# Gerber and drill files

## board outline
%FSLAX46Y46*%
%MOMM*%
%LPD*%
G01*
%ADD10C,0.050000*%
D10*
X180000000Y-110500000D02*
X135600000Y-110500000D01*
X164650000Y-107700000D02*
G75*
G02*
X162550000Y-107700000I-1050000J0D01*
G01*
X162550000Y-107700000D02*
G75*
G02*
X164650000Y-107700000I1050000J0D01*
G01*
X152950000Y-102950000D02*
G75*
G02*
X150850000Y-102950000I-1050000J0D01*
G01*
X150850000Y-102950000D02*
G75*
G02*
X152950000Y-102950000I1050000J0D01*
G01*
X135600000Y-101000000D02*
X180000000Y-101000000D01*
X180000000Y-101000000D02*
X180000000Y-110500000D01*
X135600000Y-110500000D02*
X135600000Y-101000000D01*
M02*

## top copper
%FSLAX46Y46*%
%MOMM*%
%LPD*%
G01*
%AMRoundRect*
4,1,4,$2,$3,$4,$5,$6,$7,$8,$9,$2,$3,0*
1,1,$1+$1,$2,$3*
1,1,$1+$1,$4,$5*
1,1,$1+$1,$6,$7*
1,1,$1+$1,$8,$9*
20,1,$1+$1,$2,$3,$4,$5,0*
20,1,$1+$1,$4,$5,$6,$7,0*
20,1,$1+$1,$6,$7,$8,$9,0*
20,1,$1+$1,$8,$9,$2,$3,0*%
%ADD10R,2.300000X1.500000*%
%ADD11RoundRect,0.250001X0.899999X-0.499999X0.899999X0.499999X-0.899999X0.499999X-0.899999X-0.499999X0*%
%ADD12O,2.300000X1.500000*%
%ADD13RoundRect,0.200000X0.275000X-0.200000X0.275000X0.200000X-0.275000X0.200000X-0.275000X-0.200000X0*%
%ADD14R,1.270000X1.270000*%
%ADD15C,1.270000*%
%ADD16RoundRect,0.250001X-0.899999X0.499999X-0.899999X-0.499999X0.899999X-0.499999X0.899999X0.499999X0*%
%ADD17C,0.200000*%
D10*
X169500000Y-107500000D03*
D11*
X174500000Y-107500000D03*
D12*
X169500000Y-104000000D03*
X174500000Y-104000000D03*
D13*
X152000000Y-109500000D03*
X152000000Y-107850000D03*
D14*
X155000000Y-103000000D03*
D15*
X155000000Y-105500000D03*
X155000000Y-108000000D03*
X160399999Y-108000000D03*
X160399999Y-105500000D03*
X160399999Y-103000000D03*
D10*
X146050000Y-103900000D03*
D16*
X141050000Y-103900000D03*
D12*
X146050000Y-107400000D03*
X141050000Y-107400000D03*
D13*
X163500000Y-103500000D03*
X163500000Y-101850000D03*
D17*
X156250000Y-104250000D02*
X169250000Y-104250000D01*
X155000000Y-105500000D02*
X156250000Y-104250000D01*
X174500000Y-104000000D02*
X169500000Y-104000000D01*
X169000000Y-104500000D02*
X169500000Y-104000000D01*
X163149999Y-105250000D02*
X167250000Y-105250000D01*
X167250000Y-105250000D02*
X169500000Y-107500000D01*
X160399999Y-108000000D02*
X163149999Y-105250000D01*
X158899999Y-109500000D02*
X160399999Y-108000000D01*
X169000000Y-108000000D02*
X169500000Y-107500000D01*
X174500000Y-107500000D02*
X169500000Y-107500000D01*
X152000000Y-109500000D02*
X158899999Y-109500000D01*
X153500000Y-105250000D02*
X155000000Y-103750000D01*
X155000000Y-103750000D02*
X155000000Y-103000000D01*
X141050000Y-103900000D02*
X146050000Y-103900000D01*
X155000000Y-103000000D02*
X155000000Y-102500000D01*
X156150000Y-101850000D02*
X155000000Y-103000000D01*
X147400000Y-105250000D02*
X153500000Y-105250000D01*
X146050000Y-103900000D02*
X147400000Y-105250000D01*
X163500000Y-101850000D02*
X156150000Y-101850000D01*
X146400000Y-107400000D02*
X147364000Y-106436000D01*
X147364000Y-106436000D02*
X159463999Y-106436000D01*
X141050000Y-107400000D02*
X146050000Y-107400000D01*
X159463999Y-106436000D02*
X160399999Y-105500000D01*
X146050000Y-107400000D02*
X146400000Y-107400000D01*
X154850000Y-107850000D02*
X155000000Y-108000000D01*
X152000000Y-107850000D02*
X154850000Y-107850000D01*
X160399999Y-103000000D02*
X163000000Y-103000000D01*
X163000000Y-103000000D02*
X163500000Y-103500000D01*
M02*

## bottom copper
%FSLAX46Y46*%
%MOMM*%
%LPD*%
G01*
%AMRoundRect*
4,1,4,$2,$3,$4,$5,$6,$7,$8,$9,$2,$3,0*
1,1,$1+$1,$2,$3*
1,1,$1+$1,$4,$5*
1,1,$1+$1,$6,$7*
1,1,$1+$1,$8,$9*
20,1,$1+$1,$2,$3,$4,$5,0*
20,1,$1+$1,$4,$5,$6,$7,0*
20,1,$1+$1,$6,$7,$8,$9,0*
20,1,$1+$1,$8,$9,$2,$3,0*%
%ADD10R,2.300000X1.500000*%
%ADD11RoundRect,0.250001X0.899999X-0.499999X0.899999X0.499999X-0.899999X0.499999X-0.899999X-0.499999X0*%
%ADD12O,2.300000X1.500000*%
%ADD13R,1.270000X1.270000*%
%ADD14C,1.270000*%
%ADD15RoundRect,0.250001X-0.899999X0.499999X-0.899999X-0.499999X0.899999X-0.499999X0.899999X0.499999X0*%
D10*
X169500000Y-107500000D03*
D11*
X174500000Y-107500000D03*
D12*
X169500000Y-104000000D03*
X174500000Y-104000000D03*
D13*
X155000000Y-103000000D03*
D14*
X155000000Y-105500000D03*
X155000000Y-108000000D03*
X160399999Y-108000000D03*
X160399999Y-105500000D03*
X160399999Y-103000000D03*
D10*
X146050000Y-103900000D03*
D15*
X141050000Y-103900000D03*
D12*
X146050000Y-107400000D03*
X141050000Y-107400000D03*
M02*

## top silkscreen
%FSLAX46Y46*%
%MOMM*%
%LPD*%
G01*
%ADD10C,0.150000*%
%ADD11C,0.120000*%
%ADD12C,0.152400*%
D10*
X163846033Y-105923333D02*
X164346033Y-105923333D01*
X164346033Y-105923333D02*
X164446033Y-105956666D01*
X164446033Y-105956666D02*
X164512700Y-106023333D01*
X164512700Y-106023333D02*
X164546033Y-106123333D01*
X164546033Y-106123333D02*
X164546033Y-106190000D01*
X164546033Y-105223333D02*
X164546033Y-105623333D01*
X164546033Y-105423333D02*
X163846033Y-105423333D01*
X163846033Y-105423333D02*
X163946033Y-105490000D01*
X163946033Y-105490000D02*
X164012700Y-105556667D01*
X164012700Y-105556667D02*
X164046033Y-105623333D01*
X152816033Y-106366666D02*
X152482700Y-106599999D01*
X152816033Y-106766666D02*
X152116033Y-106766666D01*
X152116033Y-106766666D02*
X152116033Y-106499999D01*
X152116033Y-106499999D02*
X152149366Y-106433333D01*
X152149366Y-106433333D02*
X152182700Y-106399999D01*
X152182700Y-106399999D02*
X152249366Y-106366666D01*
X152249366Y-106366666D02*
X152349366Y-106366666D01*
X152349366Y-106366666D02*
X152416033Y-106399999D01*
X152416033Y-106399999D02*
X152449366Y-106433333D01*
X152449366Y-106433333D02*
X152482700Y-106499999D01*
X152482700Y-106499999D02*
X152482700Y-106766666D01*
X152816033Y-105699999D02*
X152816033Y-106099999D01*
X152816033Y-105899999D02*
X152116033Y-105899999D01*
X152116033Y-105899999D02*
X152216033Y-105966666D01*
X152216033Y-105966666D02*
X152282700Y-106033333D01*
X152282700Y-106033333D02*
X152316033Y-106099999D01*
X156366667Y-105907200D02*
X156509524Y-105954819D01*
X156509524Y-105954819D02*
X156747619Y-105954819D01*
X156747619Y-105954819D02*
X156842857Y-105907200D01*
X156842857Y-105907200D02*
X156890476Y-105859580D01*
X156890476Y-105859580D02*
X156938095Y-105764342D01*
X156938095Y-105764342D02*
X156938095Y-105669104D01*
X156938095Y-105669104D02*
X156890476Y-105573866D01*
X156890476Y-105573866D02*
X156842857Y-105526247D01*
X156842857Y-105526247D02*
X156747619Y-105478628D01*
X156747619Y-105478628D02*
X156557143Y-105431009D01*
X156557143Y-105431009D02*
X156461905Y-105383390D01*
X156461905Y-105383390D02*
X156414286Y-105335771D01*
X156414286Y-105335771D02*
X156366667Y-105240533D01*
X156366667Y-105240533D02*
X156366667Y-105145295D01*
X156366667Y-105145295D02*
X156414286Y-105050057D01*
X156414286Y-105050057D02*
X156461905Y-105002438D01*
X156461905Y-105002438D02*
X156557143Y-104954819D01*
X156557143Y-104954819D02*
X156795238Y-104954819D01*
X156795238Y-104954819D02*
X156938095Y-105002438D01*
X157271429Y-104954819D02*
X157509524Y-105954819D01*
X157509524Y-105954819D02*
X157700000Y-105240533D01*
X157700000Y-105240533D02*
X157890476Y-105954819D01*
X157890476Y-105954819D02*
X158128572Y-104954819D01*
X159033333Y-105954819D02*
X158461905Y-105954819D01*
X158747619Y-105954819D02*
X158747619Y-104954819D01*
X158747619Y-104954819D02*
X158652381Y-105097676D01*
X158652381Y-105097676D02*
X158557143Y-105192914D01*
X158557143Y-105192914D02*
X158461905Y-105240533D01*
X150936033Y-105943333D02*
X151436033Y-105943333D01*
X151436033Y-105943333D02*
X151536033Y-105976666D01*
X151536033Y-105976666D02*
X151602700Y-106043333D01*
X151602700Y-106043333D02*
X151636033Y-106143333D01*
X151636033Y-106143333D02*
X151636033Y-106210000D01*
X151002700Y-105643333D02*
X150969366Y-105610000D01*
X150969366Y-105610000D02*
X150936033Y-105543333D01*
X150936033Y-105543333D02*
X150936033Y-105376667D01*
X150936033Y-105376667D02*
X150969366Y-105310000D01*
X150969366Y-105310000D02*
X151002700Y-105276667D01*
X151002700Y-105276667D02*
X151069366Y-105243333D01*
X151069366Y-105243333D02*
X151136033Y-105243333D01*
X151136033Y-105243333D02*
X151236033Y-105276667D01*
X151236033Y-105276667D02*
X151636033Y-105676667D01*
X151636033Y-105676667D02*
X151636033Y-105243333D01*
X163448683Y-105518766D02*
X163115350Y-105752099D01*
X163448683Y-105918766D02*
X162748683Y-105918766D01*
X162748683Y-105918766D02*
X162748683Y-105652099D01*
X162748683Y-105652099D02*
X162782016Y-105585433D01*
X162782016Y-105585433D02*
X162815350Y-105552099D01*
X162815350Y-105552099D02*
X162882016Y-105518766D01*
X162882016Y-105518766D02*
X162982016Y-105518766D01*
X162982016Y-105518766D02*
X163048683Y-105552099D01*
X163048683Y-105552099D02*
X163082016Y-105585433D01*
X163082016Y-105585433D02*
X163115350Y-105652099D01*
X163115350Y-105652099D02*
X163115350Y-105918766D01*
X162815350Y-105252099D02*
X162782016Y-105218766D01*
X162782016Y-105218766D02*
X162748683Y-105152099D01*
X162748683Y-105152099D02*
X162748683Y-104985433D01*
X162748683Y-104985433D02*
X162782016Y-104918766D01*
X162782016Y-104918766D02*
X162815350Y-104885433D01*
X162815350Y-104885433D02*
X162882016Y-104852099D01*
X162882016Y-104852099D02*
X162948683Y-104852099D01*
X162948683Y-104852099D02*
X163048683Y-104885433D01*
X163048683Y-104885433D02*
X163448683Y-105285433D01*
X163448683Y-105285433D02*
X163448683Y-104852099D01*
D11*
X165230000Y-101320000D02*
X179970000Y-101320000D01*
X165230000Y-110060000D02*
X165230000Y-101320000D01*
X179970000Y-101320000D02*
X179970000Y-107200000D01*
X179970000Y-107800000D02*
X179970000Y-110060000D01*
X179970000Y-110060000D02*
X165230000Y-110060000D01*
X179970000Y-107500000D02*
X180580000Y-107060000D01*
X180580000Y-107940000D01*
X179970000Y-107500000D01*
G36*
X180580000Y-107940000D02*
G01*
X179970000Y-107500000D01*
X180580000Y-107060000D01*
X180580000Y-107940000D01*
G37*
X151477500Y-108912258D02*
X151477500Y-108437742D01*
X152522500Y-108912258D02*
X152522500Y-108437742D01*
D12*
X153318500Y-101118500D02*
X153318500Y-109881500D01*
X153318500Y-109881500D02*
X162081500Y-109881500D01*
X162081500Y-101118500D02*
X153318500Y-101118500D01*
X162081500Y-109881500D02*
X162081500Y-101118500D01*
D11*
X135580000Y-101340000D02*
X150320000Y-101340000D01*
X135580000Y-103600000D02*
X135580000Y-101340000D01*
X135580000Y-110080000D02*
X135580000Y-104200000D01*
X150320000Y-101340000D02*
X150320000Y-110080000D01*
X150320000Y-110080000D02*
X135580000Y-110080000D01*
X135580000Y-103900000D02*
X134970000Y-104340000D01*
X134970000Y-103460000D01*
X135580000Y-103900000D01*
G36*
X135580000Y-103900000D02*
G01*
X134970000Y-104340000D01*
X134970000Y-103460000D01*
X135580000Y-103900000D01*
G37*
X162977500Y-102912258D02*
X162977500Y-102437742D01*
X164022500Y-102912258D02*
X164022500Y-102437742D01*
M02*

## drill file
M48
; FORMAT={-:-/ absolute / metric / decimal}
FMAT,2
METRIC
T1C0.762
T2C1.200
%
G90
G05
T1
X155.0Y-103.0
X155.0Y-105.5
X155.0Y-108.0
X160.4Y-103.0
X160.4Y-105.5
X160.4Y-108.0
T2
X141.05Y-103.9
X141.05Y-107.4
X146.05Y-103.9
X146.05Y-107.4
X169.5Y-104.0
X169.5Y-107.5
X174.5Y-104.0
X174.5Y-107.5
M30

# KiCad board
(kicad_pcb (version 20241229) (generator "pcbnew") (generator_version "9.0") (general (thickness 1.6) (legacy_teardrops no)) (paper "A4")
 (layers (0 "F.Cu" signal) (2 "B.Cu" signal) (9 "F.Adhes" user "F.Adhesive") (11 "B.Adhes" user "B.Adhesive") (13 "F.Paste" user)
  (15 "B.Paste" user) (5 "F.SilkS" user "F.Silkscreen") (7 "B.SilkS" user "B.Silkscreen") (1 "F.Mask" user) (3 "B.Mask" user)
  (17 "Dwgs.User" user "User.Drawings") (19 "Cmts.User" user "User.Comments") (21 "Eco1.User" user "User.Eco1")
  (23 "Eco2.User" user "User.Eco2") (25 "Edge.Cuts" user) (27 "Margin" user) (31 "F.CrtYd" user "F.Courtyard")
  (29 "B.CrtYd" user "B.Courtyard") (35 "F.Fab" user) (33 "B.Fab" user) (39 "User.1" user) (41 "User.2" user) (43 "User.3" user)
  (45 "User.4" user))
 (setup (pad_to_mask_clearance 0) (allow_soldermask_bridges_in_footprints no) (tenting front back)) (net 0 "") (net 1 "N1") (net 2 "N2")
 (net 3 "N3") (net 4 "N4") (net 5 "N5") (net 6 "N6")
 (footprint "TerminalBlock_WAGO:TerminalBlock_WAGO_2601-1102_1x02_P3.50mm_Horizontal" (layer "F.Cu") (at 174.5 107.5 90)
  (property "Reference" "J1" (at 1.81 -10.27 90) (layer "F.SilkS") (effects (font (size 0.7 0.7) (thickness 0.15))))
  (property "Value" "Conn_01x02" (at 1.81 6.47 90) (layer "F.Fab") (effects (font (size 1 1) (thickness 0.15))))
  (fp_line (start 6.18 -9.27) (end 6.18 5.47) (stroke (width 0.12) (type solid)) (layer "F.SilkS"))
  (fp_line (start -2.56 -9.27) (end 6.18 -9.27) (stroke (width 0.12) (type solid)) (layer "F.SilkS"))
  (fp_line (start 6.18 5.47) (end 0.3 5.47) (stroke (width 0.12) (type solid)) (layer "F.SilkS"))
  (fp_line (start -0.3 5.47) (end -2.56 5.47) (stroke (width 0.12) (type solid)) (layer "F.SilkS"))
  (fp_line (start -2.56 5.47) (end -2.56 -9.27) (stroke (width 0.12) (type solid)) (layer "F.SilkS"))
  (fp_poly (pts (xy 0 5.47) (xy 0.44 6.08) (xy -0.44 6.08)) (stroke (width 0.12) (type solid)) (fill yes) (layer "F.SilkS"))
  (pad "1" thru_hole rect (at 0 -5 90) (size 1.5 2.3) (drill 1.2) (layers "*.Cu" "*.Mask") (remove_unused_layers no) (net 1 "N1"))
  (pad "1" thru_hole roundrect (at 0 0 90) (size 1.5 2.3) (drill 1.2) (layers "*.Cu" "*.Mask") (remove_unused_layers no)
   (roundrect_rratio 0.166667) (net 1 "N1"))
  (pad "2" thru_hole oval (at 3.5 -5 90) (size 1.5 2.3) (drill 1.2) (layers "*.Cu" "*.Mask") (remove_unused_layers no) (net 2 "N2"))
  (pad "2" thru_hole oval (at 3.5 0 90) (size 1.5 2.3) (drill 1.2) (layers "*.Cu" "*.Mask") (remove_unused_layers no) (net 2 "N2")))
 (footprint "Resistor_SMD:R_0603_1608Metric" (layer "F.Cu") (at 152 108.675 90)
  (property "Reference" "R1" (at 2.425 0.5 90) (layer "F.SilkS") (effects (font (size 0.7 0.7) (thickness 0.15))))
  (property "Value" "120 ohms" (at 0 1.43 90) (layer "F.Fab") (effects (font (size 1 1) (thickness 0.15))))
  (fp_line (start -0.237258 -0.5225) (end 0.237258 -0.5225) (stroke (width 0.12) (type solid)) (layer "F.SilkS"))
  (fp_line (start -0.237258 0.5225) (end 0.237258 0.5225) (stroke (width 0.12) (type solid)) (layer "F.SilkS"))
  (pad "1" smd roundrect (at -0.825 0 90) (size 0.8 0.95) (layers "F.Cu" "F.Mask" "F.Paste") (roundrect_rratio 0.25) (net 1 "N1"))
  (pad "2" smd roundrect (at 0.825 0 90) (size 0.8 0.95) (layers "F.Cu" "F.Mask" "F.Paste") (roundrect_rratio 0.25) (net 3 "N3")))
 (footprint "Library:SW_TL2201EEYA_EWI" (layer "F.Cu") (at 155 103)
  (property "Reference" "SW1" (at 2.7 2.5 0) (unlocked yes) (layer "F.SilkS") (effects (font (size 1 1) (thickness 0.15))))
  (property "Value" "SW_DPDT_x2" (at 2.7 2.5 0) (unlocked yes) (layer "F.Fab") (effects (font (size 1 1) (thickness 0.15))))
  (fp_line (start -1.6815 -1.8815) (end -1.6815 6.8815) (stroke (width 0.1524) (type solid)) (layer "F.SilkS"))
  (fp_line (start -1.6815 6.8815) (end 7.0815 6.8815) (stroke (width 0.1524) (type solid)) (layer "F.SilkS"))
  (fp_line (start 7.0815 -1.8815) (end -1.6815 -1.8815) (stroke (width 0.1524) (type solid)) (layer "F.SilkS"))
  (fp_line (start 7.0815 6.8815) (end 7.0815 -1.8815) (stroke (width 0.1524) (type solid)) (layer "F.SilkS"))
  (pad "1" thru_hole rect (at 0 0) (size 1.27 1.27) (drill 0.762) (layers "*.Cu" "*.Mask") (remove_unused_layers no) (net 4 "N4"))
  (pad "2" thru_hole circle (at 0 2.5) (size 1.27 1.27) (drill 0.762) (layers "*.Cu" "*.Mask") (remove_unused_layers no) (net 2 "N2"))
  (pad "3" thru_hole circle (at 0 5) (size 1.27 1.27) (drill 0.762) (layers "*.Cu" "*.Mask") (remove_unused_layers no) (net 3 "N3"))
  (pad "4" thru_hole circle (at 5.399999 5) (size 1.27 1.27) (drill 0.762) (layers "*.Cu" "*.Mask") (remove_unused_layers no) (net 1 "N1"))
  (pad "5" thru_hole circle (at 5.399999 2.5) (size 1.27 1.27) (drill 0.762) (layers "*.Cu" "*.Mask") (remove_unused_layers no) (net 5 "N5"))
  (pad "6" thru_hole circle (at 5.399999 0) (size 1.27 1.27) (drill 0.762) (layers "*.Cu" "*.Mask") (remove_unused_layers no) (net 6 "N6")))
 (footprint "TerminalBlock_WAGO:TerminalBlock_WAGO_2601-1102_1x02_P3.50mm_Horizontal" (layer "F.Cu") (at 141.05 103.9 -90)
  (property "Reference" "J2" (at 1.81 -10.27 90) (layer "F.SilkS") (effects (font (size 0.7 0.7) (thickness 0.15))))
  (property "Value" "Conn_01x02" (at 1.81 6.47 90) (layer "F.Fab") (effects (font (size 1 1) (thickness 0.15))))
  (fp_line (start -2.56 5.47) (end -2.56 -9.27) (stroke (width 0.12) (type solid)) (layer "F.SilkS"))
  (fp_line (start -0.3 5.47) (end -2.56 5.47) (stroke (width 0.12) (type solid)) (layer "F.SilkS"))
  (fp_line (start 6.18 5.47) (end 0.3 5.47) (stroke (width 0.12) (type solid)) (layer "F.SilkS"))
  (fp_line (start -2.56 -9.27) (end 6.18 -9.27) (stroke (width 0.12) (type solid)) (layer "F.SilkS"))
  (fp_line (start 6.18 -9.27) (end 6.18 5.47) (stroke (width 0.12) (type solid)) (layer "F.SilkS"))
  (fp_poly (pts (xy 0 5.47) (xy 0.44 6.08) (xy -0.44 6.08)) (stroke (width 0.12) (type solid)) (fill yes) (layer "F.SilkS"))
  (pad "1" thru_hole rect (at 0 -5 270) (size 1.5 2.3) (drill 1.2) (layers "*.Cu" "*.Mask") (remove_unused_layers no) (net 4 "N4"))
  (pad "1" thru_hole roundrect (at 0 0 270) (size 1.5 2.3) (drill 1.2) (layers "*.Cu" "*.Mask") (remove_unused_layers no)
   (roundrect_rratio 0.166667) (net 4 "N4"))
  (pad "2" thru_hole oval (at 3.5 -5 270) (size 1.5 2.3) (drill 1.2) (layers "*.Cu" "*.Mask") (remove_unused_layers no) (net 5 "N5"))
  (pad "2" thru_hole oval (at 3.5 0 270) (size 1.5 2.3) (drill 1.2) (layers "*.Cu" "*.Mask") (remove_unused_layers no) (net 5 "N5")))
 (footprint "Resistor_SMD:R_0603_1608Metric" (layer "F.Cu") (at 163.5 102.675 90)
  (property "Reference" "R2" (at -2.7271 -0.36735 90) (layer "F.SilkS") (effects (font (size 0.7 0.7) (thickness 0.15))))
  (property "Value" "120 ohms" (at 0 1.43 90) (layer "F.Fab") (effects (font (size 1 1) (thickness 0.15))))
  (fp_line (start -0.237258 -0.5225) (end 0.237258 -0.5225) (stroke (width 0.12) (type solid)) (layer "F.SilkS"))
  (fp_line (start -0.237258 0.5225) (end 0.237258 0.5225) (stroke (width 0.12) (type solid)) (layer "F.SilkS"))
  (pad "1" smd roundrect (at -0.825 0 90) (size 0.8 0.95) (layers "F.Cu" "F.Mask" "F.Paste") (roundrect_rratio 0.25) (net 6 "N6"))
  (pad "2" smd roundrect (at 0.825 0 90) (size 0.8 0.95) (layers "F.Cu" "F.Mask" "F.Paste") (roundrect_rratio 0.25) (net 4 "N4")))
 (gr_line (start 180 110.5) (end 135.6 110.5) (stroke (width 0.05) (type default)) (layer "Edge.Cuts"))
 (gr_circle (center 163.6 107.7) (end 162.55 107.7) (stroke (width 0.05) (type default)) (fill no) (layer "Edge.Cuts"))
 (gr_circle (center 151.9 102.95) (end 150.85 102.95) (stroke (width 0.05) (type default)) (fill no) (layer "Edge.Cuts"))
 (gr_line (start 135.6 101) (end 180 101) (stroke (width 0.05) (type default)) (layer "Edge.Cuts"))
 (gr_line (start 180 101) (end 180 110.5) (stroke (width 0.05) (type default)) (layer "Edge.Cuts"))
 (gr_line (start 135.6 110.5) (end 135.6 101) (stroke (width 0.05) (type default)) (layer "Edge.Cuts"))
 (segment (start 156.25 104.25) (end 169.25 104.25) (width 0.2) (layer "F.Cu") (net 2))
 (segment (start 155 105.5) (end 156.25 104.25) (width 0.2) (layer "F.Cu") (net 2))
 (segment (start 174.5 104) (end 169.5 104) (width 0.2) (layer "F.Cu") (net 2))
 (segment (start 169 104.5) (end 169.5 104) (width 0.2) (layer "F.Cu") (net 2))
 (segment (start 163.149999 105.25) (end 167.25 105.25) (width 0.2) (layer "F.Cu") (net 1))
 (segment (start 167.25 105.25) (end 169.5 107.5) (width 0.2) (layer "F.Cu") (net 1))
 (segment (start 160.399999 108) (end 163.149999 105.25) (width 0.2) (layer "F.Cu") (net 1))
 (segment (start 158.899999 109.5) (end 160.399999 108) (width 0.2) (layer "F.Cu") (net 1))
 (segment (start 169 108) (end 169.5 107.5) (width 0.2) (layer "F.Cu") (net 1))
 (segment (start 174.5 107.5) (end 169.5 107.5) (width 0.2) (layer "F.Cu") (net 1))
 (segment (start 152 109.5) (end 158.899999 109.5) (width 0.2) (layer "F.Cu") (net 1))
 (segment (start 153.5 105.25) (end 155 103.75) (width 0.2) (layer "F.Cu") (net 4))
 (segment (start 155 103.75) (end 155 103) (width 0.2) (layer "F.Cu") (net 4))
 (segment (start 141.05 103.9) (end 146.05 103.9) (width 0.2) (layer "F.Cu") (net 4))
 (segment (start 155 103) (end 155 102.5) (width 0.2) (layer "F.Cu") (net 4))
 (segment (start 156.15 101.85) (end 155 103) (width 0.2) (layer "F.Cu") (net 4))
 (segment (start 147.4 105.25) (end 153.5 105.25) (width 0.2) (layer "F.Cu") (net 4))
 (segment (start 146.05 103.9) (end 147.4 105.25) (width 0.2) (layer "F.Cu") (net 4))
 (segment (start 163.5 101.85) (end 156.15 101.85) (width 0.2) (layer "F.Cu") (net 4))
 (segment (start 146.4 107.4) (end 147.364 106.436) (width 0.2) (layer "F.Cu") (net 5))
 (segment (start 147.364 106.436) (end 159.463999 106.436) (width 0.2) (layer "F.Cu") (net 5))
 (segment (start 141.05 107.4) (end 146.05 107.4) (width 0.2) (layer "F.Cu") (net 5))
 (segment (start 159.463999 106.436) (end 160.399999 105.5) (width 0.2) (layer "F.Cu") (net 5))
 (segment (start 146.05 107.4) (end 146.4 107.4) (width 0.2) (layer "F.Cu") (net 5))
 (segment (start 154.85 107.85) (end 155 108) (width 0.2) (layer "F.Cu") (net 3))
 (segment (start 152 107.85) (end 154.85 107.85) (width 0.2) (layer "F.Cu") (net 3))
 (segment (start 160.399999 103) (end 163 103) (width 0.2) (layer "F.Cu") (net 6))
 (segment (start 163 103) (end 163.5 103.5) (width 0.2) (layer "F.Cu") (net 6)))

